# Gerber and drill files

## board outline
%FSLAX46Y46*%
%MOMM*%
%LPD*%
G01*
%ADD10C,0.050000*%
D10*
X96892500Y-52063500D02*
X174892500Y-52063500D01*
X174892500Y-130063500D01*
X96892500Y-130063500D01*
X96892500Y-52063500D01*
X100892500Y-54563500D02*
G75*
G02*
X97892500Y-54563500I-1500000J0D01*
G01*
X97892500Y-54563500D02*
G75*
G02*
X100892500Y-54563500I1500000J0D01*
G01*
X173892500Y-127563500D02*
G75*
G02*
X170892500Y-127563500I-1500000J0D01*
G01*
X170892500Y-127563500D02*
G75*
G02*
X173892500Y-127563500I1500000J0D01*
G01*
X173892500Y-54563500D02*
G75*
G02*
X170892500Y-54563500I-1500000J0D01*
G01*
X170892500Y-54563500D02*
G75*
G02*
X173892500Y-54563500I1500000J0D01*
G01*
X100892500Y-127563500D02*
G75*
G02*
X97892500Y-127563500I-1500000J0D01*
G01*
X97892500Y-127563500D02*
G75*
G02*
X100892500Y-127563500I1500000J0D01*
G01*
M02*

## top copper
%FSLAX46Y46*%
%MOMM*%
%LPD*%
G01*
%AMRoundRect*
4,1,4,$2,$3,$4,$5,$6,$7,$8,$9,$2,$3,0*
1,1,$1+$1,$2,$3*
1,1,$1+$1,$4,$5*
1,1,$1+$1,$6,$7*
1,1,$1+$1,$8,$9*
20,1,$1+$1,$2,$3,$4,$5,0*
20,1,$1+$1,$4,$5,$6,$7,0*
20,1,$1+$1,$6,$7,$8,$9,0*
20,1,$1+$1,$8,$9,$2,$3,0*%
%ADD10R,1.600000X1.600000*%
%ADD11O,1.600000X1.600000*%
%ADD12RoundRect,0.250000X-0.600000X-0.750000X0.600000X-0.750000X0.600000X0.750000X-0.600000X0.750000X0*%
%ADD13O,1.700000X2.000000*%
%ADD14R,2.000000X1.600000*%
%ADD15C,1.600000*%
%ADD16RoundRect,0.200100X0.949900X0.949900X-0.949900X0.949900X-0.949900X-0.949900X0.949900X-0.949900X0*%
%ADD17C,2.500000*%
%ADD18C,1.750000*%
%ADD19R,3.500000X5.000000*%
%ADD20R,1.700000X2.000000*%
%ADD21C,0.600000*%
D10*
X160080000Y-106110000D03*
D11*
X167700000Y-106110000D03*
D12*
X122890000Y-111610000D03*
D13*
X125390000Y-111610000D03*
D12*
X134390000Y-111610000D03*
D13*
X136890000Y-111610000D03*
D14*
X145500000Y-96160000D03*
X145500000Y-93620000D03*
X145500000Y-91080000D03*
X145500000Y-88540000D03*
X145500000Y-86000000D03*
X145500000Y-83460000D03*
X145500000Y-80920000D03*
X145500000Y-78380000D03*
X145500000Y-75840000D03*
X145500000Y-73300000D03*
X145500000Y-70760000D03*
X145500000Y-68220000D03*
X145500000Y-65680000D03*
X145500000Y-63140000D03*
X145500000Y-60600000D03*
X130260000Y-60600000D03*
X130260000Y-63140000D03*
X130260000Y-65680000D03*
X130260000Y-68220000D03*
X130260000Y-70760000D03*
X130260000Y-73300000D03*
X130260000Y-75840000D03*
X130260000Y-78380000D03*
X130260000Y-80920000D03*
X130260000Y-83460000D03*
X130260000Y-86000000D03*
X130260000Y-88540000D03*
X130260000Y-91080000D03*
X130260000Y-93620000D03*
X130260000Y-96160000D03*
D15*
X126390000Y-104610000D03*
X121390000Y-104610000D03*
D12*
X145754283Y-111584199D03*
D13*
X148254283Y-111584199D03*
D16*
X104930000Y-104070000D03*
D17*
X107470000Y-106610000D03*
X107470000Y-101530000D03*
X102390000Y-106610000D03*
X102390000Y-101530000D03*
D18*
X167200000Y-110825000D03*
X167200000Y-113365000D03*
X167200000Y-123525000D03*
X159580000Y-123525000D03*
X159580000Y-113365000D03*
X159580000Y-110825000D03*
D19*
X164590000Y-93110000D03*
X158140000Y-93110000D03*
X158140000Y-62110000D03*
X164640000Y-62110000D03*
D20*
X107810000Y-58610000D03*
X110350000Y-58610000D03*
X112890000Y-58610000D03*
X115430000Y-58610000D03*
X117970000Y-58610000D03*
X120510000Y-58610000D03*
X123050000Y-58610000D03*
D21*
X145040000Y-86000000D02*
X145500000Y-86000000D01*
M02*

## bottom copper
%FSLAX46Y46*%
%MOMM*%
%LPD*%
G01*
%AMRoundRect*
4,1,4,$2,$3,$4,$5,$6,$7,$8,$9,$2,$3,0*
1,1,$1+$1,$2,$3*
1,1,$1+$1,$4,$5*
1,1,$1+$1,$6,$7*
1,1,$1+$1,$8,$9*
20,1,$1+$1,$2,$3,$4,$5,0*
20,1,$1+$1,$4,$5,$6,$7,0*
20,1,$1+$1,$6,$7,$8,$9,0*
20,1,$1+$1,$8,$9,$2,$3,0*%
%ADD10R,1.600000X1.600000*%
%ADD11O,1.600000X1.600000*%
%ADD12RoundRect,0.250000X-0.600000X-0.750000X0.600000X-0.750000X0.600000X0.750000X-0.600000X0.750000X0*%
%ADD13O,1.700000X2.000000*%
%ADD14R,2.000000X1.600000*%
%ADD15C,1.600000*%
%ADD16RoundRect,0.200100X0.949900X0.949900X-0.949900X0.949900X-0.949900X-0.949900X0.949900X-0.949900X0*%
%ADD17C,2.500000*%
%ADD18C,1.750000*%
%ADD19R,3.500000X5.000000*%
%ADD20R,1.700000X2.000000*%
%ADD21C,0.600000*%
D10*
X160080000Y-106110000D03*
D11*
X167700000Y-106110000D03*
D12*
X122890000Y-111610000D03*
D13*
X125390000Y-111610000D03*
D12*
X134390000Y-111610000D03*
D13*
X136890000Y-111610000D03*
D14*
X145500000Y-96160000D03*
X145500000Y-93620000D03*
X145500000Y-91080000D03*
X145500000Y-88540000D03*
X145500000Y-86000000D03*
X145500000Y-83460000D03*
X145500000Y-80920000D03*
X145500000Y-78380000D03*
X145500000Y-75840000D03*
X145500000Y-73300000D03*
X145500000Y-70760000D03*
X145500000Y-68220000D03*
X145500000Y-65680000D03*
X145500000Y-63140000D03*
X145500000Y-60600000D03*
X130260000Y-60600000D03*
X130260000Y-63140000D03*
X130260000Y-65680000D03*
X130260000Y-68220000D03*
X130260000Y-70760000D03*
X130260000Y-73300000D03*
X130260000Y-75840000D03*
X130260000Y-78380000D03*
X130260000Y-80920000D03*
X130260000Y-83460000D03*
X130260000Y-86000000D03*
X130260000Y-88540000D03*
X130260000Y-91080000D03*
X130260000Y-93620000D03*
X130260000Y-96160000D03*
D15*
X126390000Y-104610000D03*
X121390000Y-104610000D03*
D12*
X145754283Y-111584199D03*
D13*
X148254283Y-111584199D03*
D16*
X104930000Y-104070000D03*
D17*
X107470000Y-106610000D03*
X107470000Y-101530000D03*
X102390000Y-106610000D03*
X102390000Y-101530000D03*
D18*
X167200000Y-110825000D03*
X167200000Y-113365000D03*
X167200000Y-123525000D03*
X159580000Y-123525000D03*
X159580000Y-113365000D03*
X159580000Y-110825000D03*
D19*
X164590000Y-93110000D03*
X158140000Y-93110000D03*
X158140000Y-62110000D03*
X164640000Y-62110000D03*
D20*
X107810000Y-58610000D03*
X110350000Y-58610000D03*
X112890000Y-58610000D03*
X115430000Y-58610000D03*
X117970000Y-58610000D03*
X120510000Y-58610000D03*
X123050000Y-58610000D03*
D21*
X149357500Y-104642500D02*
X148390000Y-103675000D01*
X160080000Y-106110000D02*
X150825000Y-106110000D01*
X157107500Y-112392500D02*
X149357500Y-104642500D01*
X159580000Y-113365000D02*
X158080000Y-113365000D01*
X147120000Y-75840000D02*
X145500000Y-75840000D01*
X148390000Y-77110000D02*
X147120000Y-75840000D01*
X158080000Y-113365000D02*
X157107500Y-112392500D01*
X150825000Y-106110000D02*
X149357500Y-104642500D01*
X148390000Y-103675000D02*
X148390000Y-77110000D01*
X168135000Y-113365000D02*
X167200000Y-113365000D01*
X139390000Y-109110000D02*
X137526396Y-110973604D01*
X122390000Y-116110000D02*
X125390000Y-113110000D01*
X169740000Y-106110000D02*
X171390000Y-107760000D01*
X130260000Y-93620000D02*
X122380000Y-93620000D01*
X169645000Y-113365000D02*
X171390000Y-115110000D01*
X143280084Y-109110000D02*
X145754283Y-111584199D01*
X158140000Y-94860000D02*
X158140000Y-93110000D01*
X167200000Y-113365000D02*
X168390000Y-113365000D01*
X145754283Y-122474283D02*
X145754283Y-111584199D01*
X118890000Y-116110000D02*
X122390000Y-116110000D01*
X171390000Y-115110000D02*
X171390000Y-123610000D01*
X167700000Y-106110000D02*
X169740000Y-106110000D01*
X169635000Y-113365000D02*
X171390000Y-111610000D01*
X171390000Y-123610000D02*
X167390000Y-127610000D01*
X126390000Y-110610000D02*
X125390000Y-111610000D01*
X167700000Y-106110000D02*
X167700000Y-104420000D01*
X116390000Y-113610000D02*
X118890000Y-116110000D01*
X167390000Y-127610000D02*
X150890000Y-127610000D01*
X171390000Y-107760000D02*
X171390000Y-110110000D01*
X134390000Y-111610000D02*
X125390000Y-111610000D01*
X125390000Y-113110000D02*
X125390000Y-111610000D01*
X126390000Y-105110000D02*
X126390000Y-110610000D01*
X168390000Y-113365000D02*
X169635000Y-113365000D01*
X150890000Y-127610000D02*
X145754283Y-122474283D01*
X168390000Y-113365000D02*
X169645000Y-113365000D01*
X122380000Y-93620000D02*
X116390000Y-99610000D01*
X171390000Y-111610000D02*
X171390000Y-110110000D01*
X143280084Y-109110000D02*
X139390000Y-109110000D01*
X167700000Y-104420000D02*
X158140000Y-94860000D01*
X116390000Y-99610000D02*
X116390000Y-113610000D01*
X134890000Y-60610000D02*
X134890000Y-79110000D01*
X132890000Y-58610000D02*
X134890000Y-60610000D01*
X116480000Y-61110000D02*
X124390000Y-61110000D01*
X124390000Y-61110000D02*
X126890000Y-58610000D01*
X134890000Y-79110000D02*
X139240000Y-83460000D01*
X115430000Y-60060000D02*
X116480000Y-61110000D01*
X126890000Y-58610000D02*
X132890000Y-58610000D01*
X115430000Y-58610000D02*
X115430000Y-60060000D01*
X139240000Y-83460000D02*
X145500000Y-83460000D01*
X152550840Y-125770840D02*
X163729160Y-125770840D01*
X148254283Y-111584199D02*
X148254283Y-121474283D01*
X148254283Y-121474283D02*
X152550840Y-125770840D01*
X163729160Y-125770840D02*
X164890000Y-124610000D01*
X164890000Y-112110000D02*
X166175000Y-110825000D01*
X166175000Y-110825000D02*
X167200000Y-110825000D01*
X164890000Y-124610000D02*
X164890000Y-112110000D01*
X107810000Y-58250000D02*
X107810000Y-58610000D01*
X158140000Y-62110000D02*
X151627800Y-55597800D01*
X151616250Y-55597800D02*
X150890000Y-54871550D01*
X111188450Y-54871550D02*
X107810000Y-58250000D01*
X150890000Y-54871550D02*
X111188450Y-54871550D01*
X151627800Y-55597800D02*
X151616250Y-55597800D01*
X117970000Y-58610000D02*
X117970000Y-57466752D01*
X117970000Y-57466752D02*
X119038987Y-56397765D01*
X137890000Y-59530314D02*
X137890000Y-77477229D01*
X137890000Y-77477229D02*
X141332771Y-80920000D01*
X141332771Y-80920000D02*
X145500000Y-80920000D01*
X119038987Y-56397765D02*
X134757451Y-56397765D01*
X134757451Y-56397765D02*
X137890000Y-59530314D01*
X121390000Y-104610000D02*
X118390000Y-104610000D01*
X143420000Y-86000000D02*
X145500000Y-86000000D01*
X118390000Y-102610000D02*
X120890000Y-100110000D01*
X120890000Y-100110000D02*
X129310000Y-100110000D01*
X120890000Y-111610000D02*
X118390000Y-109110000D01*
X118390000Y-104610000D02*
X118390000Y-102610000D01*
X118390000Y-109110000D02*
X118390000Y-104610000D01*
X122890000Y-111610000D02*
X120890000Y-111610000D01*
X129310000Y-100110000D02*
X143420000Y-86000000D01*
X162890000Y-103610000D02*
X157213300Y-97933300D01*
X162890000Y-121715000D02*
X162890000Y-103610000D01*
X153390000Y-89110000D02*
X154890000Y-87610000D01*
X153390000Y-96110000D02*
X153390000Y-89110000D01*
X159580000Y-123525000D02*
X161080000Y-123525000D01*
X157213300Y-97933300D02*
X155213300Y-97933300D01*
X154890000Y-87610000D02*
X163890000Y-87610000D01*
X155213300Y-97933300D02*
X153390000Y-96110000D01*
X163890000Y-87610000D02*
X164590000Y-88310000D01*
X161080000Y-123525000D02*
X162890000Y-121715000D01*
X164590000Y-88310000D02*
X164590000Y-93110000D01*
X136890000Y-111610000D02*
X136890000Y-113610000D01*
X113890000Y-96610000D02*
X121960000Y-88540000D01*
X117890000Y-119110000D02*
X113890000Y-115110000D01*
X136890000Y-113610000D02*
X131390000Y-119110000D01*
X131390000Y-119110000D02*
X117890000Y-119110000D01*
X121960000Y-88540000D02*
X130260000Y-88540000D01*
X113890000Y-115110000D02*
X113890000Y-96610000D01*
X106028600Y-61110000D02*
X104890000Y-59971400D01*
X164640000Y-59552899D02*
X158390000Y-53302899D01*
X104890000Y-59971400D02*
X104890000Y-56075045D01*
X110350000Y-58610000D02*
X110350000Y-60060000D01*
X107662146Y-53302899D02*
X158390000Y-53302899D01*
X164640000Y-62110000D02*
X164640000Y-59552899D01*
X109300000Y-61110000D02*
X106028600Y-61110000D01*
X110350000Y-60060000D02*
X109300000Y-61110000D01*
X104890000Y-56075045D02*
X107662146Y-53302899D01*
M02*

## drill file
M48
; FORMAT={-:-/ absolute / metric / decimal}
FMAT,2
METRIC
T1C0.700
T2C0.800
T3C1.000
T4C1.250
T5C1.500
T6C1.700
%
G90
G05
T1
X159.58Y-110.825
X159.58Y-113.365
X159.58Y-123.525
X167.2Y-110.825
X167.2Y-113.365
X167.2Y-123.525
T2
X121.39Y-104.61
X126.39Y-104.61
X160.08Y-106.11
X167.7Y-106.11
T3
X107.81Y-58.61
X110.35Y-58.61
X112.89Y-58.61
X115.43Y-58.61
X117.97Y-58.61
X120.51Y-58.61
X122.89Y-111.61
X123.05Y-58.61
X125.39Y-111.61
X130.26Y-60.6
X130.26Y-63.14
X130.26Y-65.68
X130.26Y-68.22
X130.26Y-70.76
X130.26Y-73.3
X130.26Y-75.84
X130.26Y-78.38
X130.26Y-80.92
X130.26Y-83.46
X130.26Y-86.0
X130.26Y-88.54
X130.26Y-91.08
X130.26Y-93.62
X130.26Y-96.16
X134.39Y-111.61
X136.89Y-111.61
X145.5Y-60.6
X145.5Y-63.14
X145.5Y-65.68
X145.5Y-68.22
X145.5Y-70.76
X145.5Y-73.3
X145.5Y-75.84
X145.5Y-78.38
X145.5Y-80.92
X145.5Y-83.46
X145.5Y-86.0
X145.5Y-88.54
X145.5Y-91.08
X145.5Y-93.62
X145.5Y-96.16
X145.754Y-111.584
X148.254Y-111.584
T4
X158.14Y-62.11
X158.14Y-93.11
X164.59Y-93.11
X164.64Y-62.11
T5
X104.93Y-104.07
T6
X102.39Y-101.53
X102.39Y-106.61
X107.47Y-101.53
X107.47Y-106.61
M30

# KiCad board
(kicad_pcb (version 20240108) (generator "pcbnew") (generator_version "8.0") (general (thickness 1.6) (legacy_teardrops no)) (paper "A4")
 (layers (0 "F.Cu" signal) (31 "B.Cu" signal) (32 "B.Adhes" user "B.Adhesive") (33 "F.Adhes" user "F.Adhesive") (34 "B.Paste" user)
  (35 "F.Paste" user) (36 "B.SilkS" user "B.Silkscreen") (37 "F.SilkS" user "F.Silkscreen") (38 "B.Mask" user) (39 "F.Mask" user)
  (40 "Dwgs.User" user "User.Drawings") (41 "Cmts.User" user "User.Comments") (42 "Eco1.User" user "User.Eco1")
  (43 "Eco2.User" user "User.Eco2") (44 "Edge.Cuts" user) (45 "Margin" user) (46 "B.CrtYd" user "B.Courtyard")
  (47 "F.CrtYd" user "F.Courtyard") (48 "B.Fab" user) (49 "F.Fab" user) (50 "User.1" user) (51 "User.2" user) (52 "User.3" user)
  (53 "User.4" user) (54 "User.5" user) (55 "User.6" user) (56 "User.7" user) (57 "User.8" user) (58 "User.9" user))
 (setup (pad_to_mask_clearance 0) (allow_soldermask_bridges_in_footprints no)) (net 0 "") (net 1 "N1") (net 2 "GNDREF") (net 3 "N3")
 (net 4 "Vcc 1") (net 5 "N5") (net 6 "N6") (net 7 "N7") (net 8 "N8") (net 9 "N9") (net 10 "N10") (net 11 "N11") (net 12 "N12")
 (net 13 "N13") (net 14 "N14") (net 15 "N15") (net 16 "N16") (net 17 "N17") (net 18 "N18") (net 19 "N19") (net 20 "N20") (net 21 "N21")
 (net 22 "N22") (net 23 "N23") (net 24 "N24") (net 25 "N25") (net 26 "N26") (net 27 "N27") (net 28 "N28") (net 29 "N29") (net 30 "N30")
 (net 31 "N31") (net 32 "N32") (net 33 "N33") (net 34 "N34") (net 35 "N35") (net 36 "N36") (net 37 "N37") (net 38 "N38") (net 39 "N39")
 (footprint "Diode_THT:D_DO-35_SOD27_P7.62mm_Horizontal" (layer "F.Cu") (at 160.08 106.11)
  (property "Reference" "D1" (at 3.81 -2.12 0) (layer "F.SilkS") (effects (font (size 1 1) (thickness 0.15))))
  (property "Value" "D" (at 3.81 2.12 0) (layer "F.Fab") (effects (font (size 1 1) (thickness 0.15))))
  (pad "1" thru_hole rect (at 0 0) (size 1.6 1.6) (drill 0.8) (layers "*.Cu" "*.Mask") (remove_unused_layers no) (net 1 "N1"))
  (pad "2" thru_hole oval (at 7.62 0) (size 1.6 1.6) (drill 0.8) (layers "*.Cu" "*.Mask") (remove_unused_layers no) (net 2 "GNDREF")))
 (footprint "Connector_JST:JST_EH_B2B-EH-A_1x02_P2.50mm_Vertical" (layer "F.Cu") (at 122.89 111.61)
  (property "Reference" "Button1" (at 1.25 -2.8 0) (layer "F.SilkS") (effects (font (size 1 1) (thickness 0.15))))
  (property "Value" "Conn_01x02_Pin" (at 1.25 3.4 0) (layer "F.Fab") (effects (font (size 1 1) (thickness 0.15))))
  (pad "1" thru_hole roundrect (at 0 0) (size 1.7 2) (drill 1) (layers "*.Cu" "*.Mask") (remove_unused_layers no)
   (roundrect_rratio 0.147059) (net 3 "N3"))
  (pad "2" thru_hole oval (at 2.5 0) (size 1.7 2) (drill 1) (layers "*.Cu" "*.Mask") (remove_unused_layers no) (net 2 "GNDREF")))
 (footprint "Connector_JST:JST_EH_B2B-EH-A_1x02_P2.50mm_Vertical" (layer "F.Cu") (at 134.39 111.61)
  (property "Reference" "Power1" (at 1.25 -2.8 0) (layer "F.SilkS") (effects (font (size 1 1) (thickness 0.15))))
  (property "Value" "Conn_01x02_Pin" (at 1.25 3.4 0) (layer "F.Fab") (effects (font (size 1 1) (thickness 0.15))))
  (pad "1" thru_hole roundrect (at 0 0) (size 1.7 2) (drill 1) (layers "*.Cu" "*.Mask") (remove_unused_layers no)
   (roundrect_rratio 0.147059) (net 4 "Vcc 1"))
  (pad "2" thru_hole oval (at 2.5 0) (size 1.7 2) (drill 1) (layers "*.Cu" "*.Mask") (remove_unused_layers no) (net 2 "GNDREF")))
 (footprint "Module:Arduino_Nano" (layer "F.Cu") (at 145.5 96.16 180)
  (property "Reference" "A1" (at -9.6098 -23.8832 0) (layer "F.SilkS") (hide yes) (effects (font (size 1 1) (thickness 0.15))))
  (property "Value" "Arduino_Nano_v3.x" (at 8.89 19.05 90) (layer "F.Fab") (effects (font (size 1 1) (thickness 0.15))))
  (pad "1" thru_hole rect (at 0 0 180) (size 2 1.6) (drill 1) (layers "*.Cu" "*.Mask") (remove_unused_layers no) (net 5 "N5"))
  (pad "2" thru_hole rect (at 0 2.54 180) (size 2 1.6) (drill 1) (layers "*.Cu" "*.Mask") (remove_unused_layers no) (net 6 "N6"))
  (pad "3" thru_hole rect (at 0 5.08 180) (size 2 1.6) (drill 1) (layers "*.Cu" "*.Mask") (remove_unused_layers no) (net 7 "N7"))
  (pad "4" thru_hole rect (at 0 7.62 180) (size 2 1.6) (drill 1) (layers "*.Cu" "*.Mask") (remove_unused_layers no) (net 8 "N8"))
  (pad "5" thru_hole rect (at 0 10.16 180) (size 2 1.6) (drill 1) (layers "*.Cu" "*.Mask") (remove_unused_layers no) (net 3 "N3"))
  (pad "6" thru_hole rect (at 0 12.7 180) (size 2 1.6) (drill 1) (layers "*.Cu" "*.Mask") (remove_unused_layers no) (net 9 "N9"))
  (pad "7" thru_hole rect (at 0 15.24 180) (size 2 1.6) (drill 1) (layers "*.Cu" "*.Mask") (remove_unused_layers no) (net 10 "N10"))
  (pad "8" thru_hole rect (at 0 17.78 180) (size 2 1.6) (drill 1) (layers "*.Cu" "*.Mask") (remove_unused_layers no) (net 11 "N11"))
  (pad "9" thru_hole rect (at 0 20.32 180) (size 2 1.6) (drill 1) (layers "*.Cu" "*.Mask") (remove_unused_layers no) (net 1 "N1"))
  (pad "10" thru_hole rect (at 0 22.86 180) (size 2 1.6) (drill 1) (layers "*.Cu" "*.Mask") (remove_unused_layers no) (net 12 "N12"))
  (pad "11" thru_hole rect (at 0 25.4 180) (size 2 1.6) (drill 1) (layers "*.Cu" "*.Mask") (remove_unused_layers no) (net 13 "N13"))
  (pad "12" thru_hole rect (at 0 27.94 180) (size 2 1.6) (drill 1) (layers "*.Cu" "*.Mask") (remove_unused_layers no) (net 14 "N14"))
  (pad "13" thru_hole rect (at 0 30.48 180) (size 2 1.6) (drill 1) (layers "*.Cu" "*.Mask") (remove_unused_layers no) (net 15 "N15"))
  (pad "14" thru_hole rect (at 0 33.02 180) (size 2 1.6) (drill 1) (layers "*.Cu" "*.Mask") (remove_unused_layers no) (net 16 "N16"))
  (pad "15" thru_hole rect (at 0 35.56 180) (size 2 1.6) (drill 1) (layers "*.Cu" "*.Mask" "Dwgs.User") (remove_unused_layers no)
   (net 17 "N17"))
  (pad "16" thru_hole rect (at 15.24 35.56 180) (size 2 1.6) (drill 1) (layers "*.Cu" "*.Mask" "Eco1.User") (remove_unused_layers no)
   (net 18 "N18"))
  (pad "17" thru_hole rect (at 15.24 33.02 180) (size 2 1.6) (drill 1) (layers "*.Cu" "*.Mask") (remove_unused_layers no) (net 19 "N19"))
  (pad "18" thru_hole rect (at 15.24 30.48 180) (size 2 1.6) (drill 1) (layers "*.Cu" "*.Mask") (remove_unused_layers no) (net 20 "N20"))
  (pad "19" thru_hole rect (at 15.24 27.94 180) (size 2 1.6) (drill 1) (layers "*.Cu" "*.Mask") (remove_unused_layers no) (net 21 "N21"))
  (pad "20" thru_hole rect (at 15.24 25.4 180) (size 2 1.6) (drill 1) (layers "*.Cu" "*.Mask") (remove_unused_layers no) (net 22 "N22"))
  (pad "21" thru_hole rect (at 15.24 22.86 180) (size 2 1.6) (drill 1) (layers "*.Cu" "*.Mask") (remove_unused_layers no) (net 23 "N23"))
  (pad "22" thru_hole rect (at 15.24 20.32 180) (size 2 1.6) (drill 1) (layers "*.Cu" "*.Mask") (remove_unused_layers no) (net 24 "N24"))
  (pad "23" thru_hole rect (at 15.24 17.78 180) (size 2 1.6) (drill 1) (layers "*.Cu" "*.Mask") (remove_unused_layers no) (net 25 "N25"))
  (pad "24" thru_hole rect (at 15.24 15.24 180) (size 2 1.6) (drill 1) (layers "*.Cu" "*.Mask") (remove_unused_layers no) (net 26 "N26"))
  (pad "25" thru_hole rect (at 15.24 12.7 180) (size 2 1.6) (drill 1) (layers "*.Cu" "*.Mask") (remove_unused_layers no) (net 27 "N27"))
  (pad "26" thru_hole rect (at 15.24 10.16 180) (size 2 1.6) (drill 1) (layers "*.Cu" "*.Mask") (remove_unused_layers no) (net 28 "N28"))
  (pad "27" thru_hole rect (at 15.24 7.62 180) (size 2 1.6) (drill 1) (layers "*.Cu" "*.Mask") (remove_unused_layers no) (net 4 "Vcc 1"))
  (pad "28" thru_hole rect (at 15.24 5.08 180) (size 2 1.6) (drill 1) (layers "*.Cu" "*.Mask") (remove_unused_layers no) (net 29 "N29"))
  (pad "29" thru_hole rect (at 15.24 2.54 180) (size 2 1.6) (drill 1) (layers "*.Cu" "*.Mask") (remove_unused_layers no) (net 2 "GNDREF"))
  (pad "30" thru_hole rect (at 15.24 0 180) (size 2 1.6) (drill 1) (layers "*.Cu" "*.Mask") (remove_unused_layers no) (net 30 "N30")))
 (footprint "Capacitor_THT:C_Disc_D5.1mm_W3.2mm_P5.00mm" (layer "F.Cu") (at 126.39 104.61 180)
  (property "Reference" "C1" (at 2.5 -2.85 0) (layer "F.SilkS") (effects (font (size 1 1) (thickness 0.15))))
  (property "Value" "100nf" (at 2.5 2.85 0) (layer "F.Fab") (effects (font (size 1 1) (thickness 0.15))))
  (pad "1" thru_hole circle (at 0 0 180) (size 1.6 1.6) (drill 0.8) (layers "*.Cu" "*.Mask") (remove_unused_layers no) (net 2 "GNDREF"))
  (pad "2" thru_hole circle (at 5 0 180) (size 1.6 1.6) (drill 0.8) (layers "*.Cu" "*.Mask") (remove_unused_layers no) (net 3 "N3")))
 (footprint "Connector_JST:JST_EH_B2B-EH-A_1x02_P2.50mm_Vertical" (layer "F.Cu") (at 145.754283 111.584199)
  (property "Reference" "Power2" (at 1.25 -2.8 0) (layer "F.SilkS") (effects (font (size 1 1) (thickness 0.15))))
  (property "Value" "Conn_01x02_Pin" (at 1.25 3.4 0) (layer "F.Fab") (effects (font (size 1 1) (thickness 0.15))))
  (pad "1" thru_hole roundrect (at 0 0) (size 1.7 2) (drill 1) (layers "*.Cu" "*.Mask") (remove_unused_layers no)
   (roundrect_rratio 0.147059) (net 2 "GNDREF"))
  (pad "2" thru_hole oval (at 2.5 0) (size 1.7 2) (drill 1) (layers "*.Cu" "*.Mask") (remove_unused_layers no) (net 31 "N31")))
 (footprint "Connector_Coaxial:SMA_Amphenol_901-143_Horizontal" (layer "F.Cu") (at 104.93 104.07 180)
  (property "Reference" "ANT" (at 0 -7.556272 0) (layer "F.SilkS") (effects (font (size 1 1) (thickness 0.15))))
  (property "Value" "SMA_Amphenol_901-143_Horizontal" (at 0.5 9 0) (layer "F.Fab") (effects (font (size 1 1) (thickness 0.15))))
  (pad "1" thru_hole roundrect (at 0 0 180) (size 2.3 2.3) (drill 1.5) (layers "*.Cu" "*.Mask") (remove_unused_layers yes)
   (keep_end_layers yes) (zone_layer_connections) (roundrect_rratio 0.087))
  (pad "2" thru_hole circle (at -2.54 -2.54 180) (size 2.5 2.5) (drill 1.7) (layers "*.Cu" "*.Mask") (remove_unused_layers yes)
   (keep_end_layers yes) (zone_layer_connections))
  (pad "2" thru_hole circle (at -2.54 2.54 180) (size 2.5 2.5) (drill 1.7) (layers "*.Cu" "*.Mask") (remove_unused_layers yes)
   (keep_end_layers yes) (zone_layer_connections))
  (pad "2" thru_hole circle (at 2.54 -2.54 180) (size 2.5 2.5) (drill 1.7) (layers "*.Cu" "*.Mask") (remove_unused_layers yes)
   (keep_end_layers yes) (zone_layer_connections))
  (pad "2" thru_hole circle (at 2.54 2.54 180) (size 2.5 2.5) (drill 1.7) (layers "*.Cu" "*.Mask") (remove_unused_layers yes)
   (keep_end_layers yes) (zone_layer_connections)))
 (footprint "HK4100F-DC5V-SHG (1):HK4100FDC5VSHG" (layer "F.Cu") (at 167.2 110.825 -90)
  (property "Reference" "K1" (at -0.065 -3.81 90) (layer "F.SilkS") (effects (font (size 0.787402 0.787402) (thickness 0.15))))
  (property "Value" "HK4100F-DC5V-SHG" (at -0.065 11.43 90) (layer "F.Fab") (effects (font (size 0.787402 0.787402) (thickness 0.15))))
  (pad "1" thru_hole circle (at 0 0 270) (size 1.75 1.75) (drill 0.7) (layers "*.Cu" "*.Mask") (remove_unused_layers no) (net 31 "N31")
   (solder_mask_margin 0.102))
  (pad "2" thru_hole circle (at 2.54 0 270) (size 1.75 1.75) (drill 0.7) (layers "*.Cu" "*.Mask") (remove_unused_layers no) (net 2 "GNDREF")
   (solder_mask_margin 0.102))
  (pad "3" thru_hole circle (at 12.7 0 270) (size 1.75 1.75) (drill 0.7) (layers "*.Cu" "*.Mask") (remove_unused_layers no) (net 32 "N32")
   (solder_mask_margin 0.102))
  (pad "4" thru_hole circle (at 12.7 7.62 270) (size 1.75 1.75) (drill 0.7) (layers "*.Cu" "*.Mask") (remove_unused_layers no)
   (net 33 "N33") (solder_mask_margin 0.102))
  (pad "5" thru_hole circle (at 2.54 7.62 270) (size 1.75 1.75) (drill 0.7) (layers "*.Cu" "*.Mask") (remove_unused_layers no) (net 1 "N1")
   (solder_mask_margin 0.102))
  (pad "6" thru_hole circle (at 0 7.62 270) (size 1.75 1.75) (drill 0.7) (layers "*.Cu" "*.Mask") (remove_unused_layers no) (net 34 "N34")
   (solder_mask_margin 0.102)))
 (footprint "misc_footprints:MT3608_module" (layer "F.Cu") (at 161.39 79.11 -90)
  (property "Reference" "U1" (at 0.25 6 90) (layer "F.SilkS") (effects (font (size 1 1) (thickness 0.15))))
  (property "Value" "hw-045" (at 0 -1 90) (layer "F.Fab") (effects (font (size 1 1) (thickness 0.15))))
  (pad "1" thru_hole rect (at 14 -3.2 90) (size 5 3.5) (drill 1.25) (layers "*.Cu" "*.Mask" "B.SilkS") (remove_unused_layers no)
   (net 33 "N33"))
  (pad "2" thru_hole rect (at 14 3.25 90) (size 5 3.5) (drill 1.25) (layers "*.Cu" "*.Mask" "B.SilkS") (remove_unused_layers no)
   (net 2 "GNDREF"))
  (pad "3" thru_hole rect (at -17 3.25 90) (size 5 3.5) (drill 1.25) (layers "*.Cu" "*.Mask" "B.SilkS") (remove_unused_layers no)
   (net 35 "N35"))
  (pad "4" thru_hole rect (at -17 -3.25 90) (size 5 3.5) (drill 1.25) (layers "*.Cu" "*.Mask" "B.SilkS") (remove_unused_layers no)
   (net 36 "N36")))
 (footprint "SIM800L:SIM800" (layer "F.Cu") (at 109.89 73.11)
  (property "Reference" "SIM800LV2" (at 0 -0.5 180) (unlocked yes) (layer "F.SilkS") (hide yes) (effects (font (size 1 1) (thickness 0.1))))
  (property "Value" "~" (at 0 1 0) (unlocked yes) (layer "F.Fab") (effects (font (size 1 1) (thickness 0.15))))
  (pad "1" thru_hole rect (at -2.08 -14.5 90) (size 2 1.7) (drill 1) (layers "*.Cu" "B.Mask") (remove_unused_layers no) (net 35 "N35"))
  (pad "2" thru_hole rect (at 0.46 -14.5 90) (size 2 1.7) (drill 1) (layers "*.Cu" "*.Mask") (remove_unused_layers no) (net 36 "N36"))
  (pad "3" thru_hole rect (at 3 -14.5 90) (size 2 1.7) (drill 1) (layers "*.Cu" "*.Mask") (remove_unused_layers no) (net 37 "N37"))
  (pad "4" thru_hole rect (at 5.54 -14.5 90) (size 2 1.7) (drill 1) (layers "*.Cu" "*.Mask") (remove_unused_layers no) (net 9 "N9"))
  (pad "5" thru_hole rect (at 8.08 -14.5 90) (size 2 1.7) (drill 1) (layers "*.Cu" "*.Mask") (remove_unused_layers no) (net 10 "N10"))
  (pad "6" thru_hole rect (at 10.62 -14.5 90) (size 2 1.7) (drill 1) (layers "*.Cu" "*.Mask") (remove_unused_layers no) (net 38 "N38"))
  (pad "7" thru_hole rect (at 13.16 -14.5 90) (size 2 1.7) (drill 1) (layers "*.Cu" "F.Mask") (remove_unused_layers no) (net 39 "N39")))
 (gr_rect (start 96.8925 52.0635) (end 174.8925 130.0635) (stroke (width 0.05) (type default)) (fill none) (layer "Edge.Cuts"))
 (gr_circle (center 99.3925 54.5635) (end 100.8925 54.5635) (stroke (width 0.05) (type default)) (fill none) (layer "Edge.Cuts"))
 (gr_circle (center 172.3925 127.5635) (end 173.8925 127.5635) (stroke (width 0.05) (type default)) (fill none) (layer "Edge.Cuts"))
 (gr_circle (center 172.3925 54.5635) (end 173.8925 54.5635) (stroke (width 0.05) (type default)) (fill none) (layer "Edge.Cuts"))
 (gr_circle (center 99.3925 127.5635) (end 100.8925 127.5635) (stroke (width 0.05) (type default)) (fill none) (layer "Edge.Cuts"))
 (segment (start 149.3575 104.6425) (end 148.39 103.675) (width 0.6) (layer "B.Cu") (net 1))
 (segment (start 160.08 106.11) (end 150.825 106.11) (width 0.6) (layer "B.Cu") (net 1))
 (segment (start 157.1075 112.3925) (end 149.3575 104.6425) (width 0.6) (layer "B.Cu") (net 1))
 (segment (start 159.58 113.365) (end 158.08 113.365) (width 0.6) (layer "B.Cu") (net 1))
 (segment (start 147.12 75.84) (end 145.5 75.84) (width 0.6) (layer "B.Cu") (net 1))
 (segment (start 148.39 77.11) (end 147.12 75.84) (width 0.6) (layer "B.Cu") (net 1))
 (segment (start 158.08 113.365) (end 157.1075 112.3925) (width 0.6) (layer "B.Cu") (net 1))
 (segment (start 150.825 106.11) (end 149.3575 104.6425) (width 0.6) (layer "B.Cu") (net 1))
 (segment (start 148.39 103.675) (end 148.39 77.11) (width 0.6) (layer "B.Cu") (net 1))
 (segment (start 168.135 113.365) (end 167.2 113.365) (width 0.6) (layer "B.Cu") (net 2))
 (segment (start 139.39 109.11) (end 137.526396 110.973604) (width 0.6) (layer "B.Cu") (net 2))
 (segment (start 122.39 116.11) (end 125.39 113.11) (width 0.6) (layer "B.Cu") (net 2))
 (segment (start 169.74 106.11) (end 171.39 107.76) (width 0.6) (layer "B.Cu") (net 2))
 (segment (start 130.26 93.62) (end 122.38 93.62) (width 0.6) (layer "B.Cu") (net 2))
 (segment (start 169.645 113.365) (end 171.39 115.11) (width 0.6) (layer "B.Cu") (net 2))
 (segment (start 143.280084 109.11) (end 145.754283 111.584199) (width 0.6) (layer "B.Cu") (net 2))
 (segment (start 158.14 94.86) (end 158.14 93.11) (width 0.6) (layer "B.Cu") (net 2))
 (segment (start 167.2 113.365) (end 168.39 113.365) (width 0.6) (layer "B.Cu") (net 2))
 (segment (start 145.754283 122.474283) (end 145.754283 111.584199) (width 0.6) (layer "B.Cu") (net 2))
 (segment (start 118.89 116.11) (end 122.39 116.11) (width 0.6) (layer "B.Cu") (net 2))
 (segment (start 171.39 115.11) (end 171.39 123.61) (width 0.6) (layer "B.Cu") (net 2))
 (segment (start 167.7 106.11) (end 169.74 106.11) (width 0.6) (layer "B.Cu") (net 2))
 (segment (start 169.635 113.365) (end 171.39 111.61) (width 0.6) (layer "B.Cu") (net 2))
 (segment (start 171.39 123.61) (end 167.39 127.61) (width 0.6) (layer "B.Cu") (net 2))
 (segment (start 126.39 110.61) (end 125.39 111.61) (width 0.6) (layer "B.Cu") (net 2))
 (segment (start 167.7 106.11) (end 167.7 104.42) (width 0.6) (layer "B.Cu") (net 2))
 (segment (start 116.39 113.61) (end 118.89 116.11) (width 0.6) (layer "B.Cu") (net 2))
 (segment (start 167.39 127.61) (end 150.89 127.61) (width 0.6) (layer "B.Cu") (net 2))
 (segment (start 171.39 107.76) (end 171.39 110.11) (width 0.6) (layer "B.Cu") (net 2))
 (segment (start 134.39 111.61) (end 125.39 111.61) (width 0.6) (layer "B.Cu") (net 2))
 (segment (start 125.39 113.11) (end 125.39 111.61) (width 0.6) (layer "B.Cu") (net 2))
 (segment (start 126.39 105.11) (end 126.39 110.61) (width 0.6) (layer "B.Cu") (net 2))
 (segment (start 168.39 113.365) (end 169.635 113.365) (width 0.6) (layer "B.Cu") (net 2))
 (segment (start 150.89 127.61) (end 145.754283 122.474283) (width 0.6) (layer "B.Cu") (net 2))
 (segment (start 168.39 113.365) (end 169.645 113.365) (width 0.6) (layer "B.Cu") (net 2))
 (segment (start 122.38 93.62) (end 116.39 99.61) (width 0.6) (layer "B.Cu") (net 2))
 (segment (start 171.39 111.61) (end 171.39 110.11) (width 0.6) (layer "B.Cu") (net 2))
 (segment (start 143.280084 109.11) (end 139.39 109.11) (width 0.6) (layer "B.Cu") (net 2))
 (segment (start 167.7 104.42) (end 158.14 94.86) (width 0.6) (layer "B.Cu") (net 2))
 (segment (start 116.39 99.61) (end 116.39 113.61) (width 0.6) (layer "B.Cu") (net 2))
 (segment (start 134.89 60.61) (end 134.89 79.11) (width 0.6) (layer "B.Cu") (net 9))
 (segment (start 132.89 58.61) (end 134.89 60.61) (width 0.6) (layer "B.Cu") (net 9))
 (segment (start 116.48 61.11) (end 124.39 61.11) (width 0.6) (layer "B.Cu") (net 9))
 (segment (start 124.39 61.11) (end 126.89 58.61) (width 0.6) (layer "B.Cu") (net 9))
 (segment (start 134.89 79.11) (end 139.24 83.46) (width 0.6) (layer "B.Cu") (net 9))
 (segment (start 115.43 60.06) (end 116.48 61.11) (width 0.6) (layer "B.Cu") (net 9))
 (segment (start 126.89 58.61) (end 132.89 58.61) (width 0.6) (layer "B.Cu") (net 9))
 (segment (start 115.43 58.61) (end 115.43 60.06) (width 0.6) (layer "B.Cu") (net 9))
 (segment (start 139.24 83.46) (end 145.5 83.46) (width 0.6) (layer "B.Cu") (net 9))
 (segment (start 152.55084 125.77084) (end 163.72916 125.77084) (width 0.6) (layer "B.Cu") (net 31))
 (segment (start 148.254283 111.584199) (end 148.254283 121.474283) (width 0.6) (layer "B.Cu") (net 31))
 (segment (start 148.254283 121.474283) (end 152.55084 125.77084) (width 0.6) (layer "B.Cu") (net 31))
 (segment (start 163.72916 125.77084) (end 164.89 124.61) (width 0.6) (layer "B.Cu") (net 31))
 (segment (start 164.89 112.11) (end 166.175 110.825) (width 0.6) (layer "B.Cu") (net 31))
 (segment (start 166.175 110.825) (end 167.2 110.825) (width 0.6) (layer "B.Cu") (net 31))
 (segment (start 164.89 124.61) (end 164.89 112.11) (width 0.6) (layer "B.Cu") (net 31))
 (segment (start 107.81 58.25) (end 107.81 58.61) (width 0.6) (layer "B.Cu") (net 35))
 (segment (start 158.14 62.11) (end 151.6278 55.5978) (width 0.6) (layer "B.Cu") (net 35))
 (segment (start 151.61625 55.5978) (end 150.89 54.87155) (width 0.6) (layer "B.Cu") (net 35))
 (segment (start 111.18845 54.87155) (end 107.81 58.25) (width 0.6) (layer "B.Cu") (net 35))
 (segment (start 150.89 54.87155) (end 111.18845 54.87155) (width 0.6) (layer "B.Cu") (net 35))
 (segment (start 151.6278 55.5978) (end 151.61625 55.5978) (width 0.6) (layer "B.Cu") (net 35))
 (segment (start 117.97 58.61) (end 117.97 57.466752) (width 0.6) (layer "B.Cu") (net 10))
 (segment (start 117.97 57.466752) (end 119.038987 56.397765) (width 0.6) (layer "B.Cu") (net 10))
 (segment (start 137.89 59.530314) (end 137.89 77.477229) (width 0.6) (layer "B.Cu") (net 10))
 (segment (start 137.89 77.477229) (end 141.332771 80.92) (width 0.6) (layer "B.Cu") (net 10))
 (segment (start 141.332771 80.92) (end 145.5 80.92) (width 0.6) (layer "B.Cu") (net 10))
 (segment (start 119.038987 56.397765) (end 134.757451 56.397765) (width 0.6) (layer "B.Cu") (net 10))
 (segment (start 134.757451 56.397765) (end 137.89 59.530314) (width 0.6) (layer "B.Cu") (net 10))
 (segment (start 145.04 86) (end 145.5 86) (width 0.6) (layer "F.Cu") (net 3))
 (segment (start 121.39 104.61) (end 118.39 104.61) (width 0.6) (layer "B.Cu") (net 3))
 (segment (start 143.42 86) (end 145.5 86) (width 0.6) (layer "B.Cu") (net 3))
 (segment (start 118.39 102.61) (end 120.89 100.11) (width 0.6) (layer "B.Cu") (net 3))
 (segment (start 120.89 100.11) (end 129.31 100.11) (width 0.6) (layer "B.Cu") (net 3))
 (segment (start 120.89 111.61) (end 118.39 109.11) (width 0.6) (layer "B.Cu") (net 3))
 (segment (start 118.39 104.61) (end 118.39 102.61) (width 0.6) (layer "B.Cu") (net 3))
 (segment (start 118.39 109.11) (end 118.39 104.61) (width 0.6) (layer "B.Cu") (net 3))
 (segment (start 122.89 111.61) (end 120.89 111.61) (width 0.6) (layer "B.Cu") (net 3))
 (segment (start 129.31 100.11) (end 143.42 86) (width 0.6) (layer "B.Cu") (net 3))
 (segment (start 162.89 103.61) (end 157.2133 97.9333) (width 0.6) (layer "B.Cu") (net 33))
 (segment (start 162.89 121.715) (end 162.89 103.61) (width 0.6) (layer "B.Cu") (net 33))
 (segment (start 153.39 89.11) (end 154.89 87.61) (width 0.6) (layer "B.Cu") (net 33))
 (segment (start 153.39 96.11) (end 153.39 89.11) (width 0.6) (layer "B.Cu") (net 33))
 (segment (start 159.58 123.525) (end 161.08 123.525) (width 0.6) (layer "B.Cu") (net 33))
 (segment (start 157.2133 97.9333) (end 155.2133 97.9333) (width 0.6) (layer "B.Cu") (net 33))
 (segment (start 154.89 87.61) (end 163.89 87.61) (width 0.6) (layer "B.Cu") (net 33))
 (segment (start 155.2133 97.9333) (end 153.39 96.11) (width 0.6) (layer "B.Cu") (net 33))
 (segment (start 163.89 87.61) (end 164.59 88.31) (width 0.6) (layer "B.Cu") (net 33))
 (segment (start 161.08 123.525) (end 162.89 121.715) (width 0.6) (layer "B.Cu") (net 33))
 (segment (start 164.59 88.31) (end 164.59 93.11) (width 0.6) (layer "B.Cu") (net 33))
 (segment (start 136.89 111.61) (end 136.89 113.61) (width 0.6) (layer "B.Cu") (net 4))
 (segment (start 113.89 96.61) (end 121.96 88.54) (width 0.6) (layer "B.Cu") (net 4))
 (segment (start 117.89 119.11) (end 113.89 115.11) (width 0.6) (layer "B.Cu") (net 4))
 (segment (start 136.89 113.61) (end 131.39 119.11) (width 0.6) (layer "B.Cu") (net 4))
 (segment (start 131.39 119.11) (end 117.89 119.11) (width 0.6) (layer "B.Cu") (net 4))
 (segment (start 121.96 88.54) (end 130.26 88.54) (width 0.6) (layer "B.Cu") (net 4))
 (segment (start 113.89 115.11) (end 113.89 96.61) (width 0.6) (layer "B.Cu") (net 4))
 (segment (start 106.0286 61.11) (end 104.89 59.9714) (width 0.6) (layer "B.Cu") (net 36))
 (segment (start 164.64 59.552899) (end 158.39 53.302899) (width 0.6) (layer "B.Cu") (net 36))
 (segment (start 104.89 59.9714) (end 104.89 56.075045) (width 0.6) (layer "B.Cu") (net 36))
 (segment (start 110.35 58.61) (end 110.35 60.06) (width 0.6) (layer "B.Cu") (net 36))
 (segment (start 107.662146 53.302899) (end 158.39 53.302899) (width 0.6) (layer "B.Cu") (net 36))
 (segment (start 164.64 62.11) (end 164.64 59.552899) (width 0.6) (layer "B.Cu") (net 36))
 (segment (start 109.3 61.11) (end 106.0286 61.11) (width 0.6) (layer "B.Cu") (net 36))
 (segment (start 110.35 60.06) (end 109.3 61.11) (width 0.6) (layer "B.Cu") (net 36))
 (segment (start 104.89 56.075045) (end 107.662146 53.302899) (width 0.6) (layer "B.Cu") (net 36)))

